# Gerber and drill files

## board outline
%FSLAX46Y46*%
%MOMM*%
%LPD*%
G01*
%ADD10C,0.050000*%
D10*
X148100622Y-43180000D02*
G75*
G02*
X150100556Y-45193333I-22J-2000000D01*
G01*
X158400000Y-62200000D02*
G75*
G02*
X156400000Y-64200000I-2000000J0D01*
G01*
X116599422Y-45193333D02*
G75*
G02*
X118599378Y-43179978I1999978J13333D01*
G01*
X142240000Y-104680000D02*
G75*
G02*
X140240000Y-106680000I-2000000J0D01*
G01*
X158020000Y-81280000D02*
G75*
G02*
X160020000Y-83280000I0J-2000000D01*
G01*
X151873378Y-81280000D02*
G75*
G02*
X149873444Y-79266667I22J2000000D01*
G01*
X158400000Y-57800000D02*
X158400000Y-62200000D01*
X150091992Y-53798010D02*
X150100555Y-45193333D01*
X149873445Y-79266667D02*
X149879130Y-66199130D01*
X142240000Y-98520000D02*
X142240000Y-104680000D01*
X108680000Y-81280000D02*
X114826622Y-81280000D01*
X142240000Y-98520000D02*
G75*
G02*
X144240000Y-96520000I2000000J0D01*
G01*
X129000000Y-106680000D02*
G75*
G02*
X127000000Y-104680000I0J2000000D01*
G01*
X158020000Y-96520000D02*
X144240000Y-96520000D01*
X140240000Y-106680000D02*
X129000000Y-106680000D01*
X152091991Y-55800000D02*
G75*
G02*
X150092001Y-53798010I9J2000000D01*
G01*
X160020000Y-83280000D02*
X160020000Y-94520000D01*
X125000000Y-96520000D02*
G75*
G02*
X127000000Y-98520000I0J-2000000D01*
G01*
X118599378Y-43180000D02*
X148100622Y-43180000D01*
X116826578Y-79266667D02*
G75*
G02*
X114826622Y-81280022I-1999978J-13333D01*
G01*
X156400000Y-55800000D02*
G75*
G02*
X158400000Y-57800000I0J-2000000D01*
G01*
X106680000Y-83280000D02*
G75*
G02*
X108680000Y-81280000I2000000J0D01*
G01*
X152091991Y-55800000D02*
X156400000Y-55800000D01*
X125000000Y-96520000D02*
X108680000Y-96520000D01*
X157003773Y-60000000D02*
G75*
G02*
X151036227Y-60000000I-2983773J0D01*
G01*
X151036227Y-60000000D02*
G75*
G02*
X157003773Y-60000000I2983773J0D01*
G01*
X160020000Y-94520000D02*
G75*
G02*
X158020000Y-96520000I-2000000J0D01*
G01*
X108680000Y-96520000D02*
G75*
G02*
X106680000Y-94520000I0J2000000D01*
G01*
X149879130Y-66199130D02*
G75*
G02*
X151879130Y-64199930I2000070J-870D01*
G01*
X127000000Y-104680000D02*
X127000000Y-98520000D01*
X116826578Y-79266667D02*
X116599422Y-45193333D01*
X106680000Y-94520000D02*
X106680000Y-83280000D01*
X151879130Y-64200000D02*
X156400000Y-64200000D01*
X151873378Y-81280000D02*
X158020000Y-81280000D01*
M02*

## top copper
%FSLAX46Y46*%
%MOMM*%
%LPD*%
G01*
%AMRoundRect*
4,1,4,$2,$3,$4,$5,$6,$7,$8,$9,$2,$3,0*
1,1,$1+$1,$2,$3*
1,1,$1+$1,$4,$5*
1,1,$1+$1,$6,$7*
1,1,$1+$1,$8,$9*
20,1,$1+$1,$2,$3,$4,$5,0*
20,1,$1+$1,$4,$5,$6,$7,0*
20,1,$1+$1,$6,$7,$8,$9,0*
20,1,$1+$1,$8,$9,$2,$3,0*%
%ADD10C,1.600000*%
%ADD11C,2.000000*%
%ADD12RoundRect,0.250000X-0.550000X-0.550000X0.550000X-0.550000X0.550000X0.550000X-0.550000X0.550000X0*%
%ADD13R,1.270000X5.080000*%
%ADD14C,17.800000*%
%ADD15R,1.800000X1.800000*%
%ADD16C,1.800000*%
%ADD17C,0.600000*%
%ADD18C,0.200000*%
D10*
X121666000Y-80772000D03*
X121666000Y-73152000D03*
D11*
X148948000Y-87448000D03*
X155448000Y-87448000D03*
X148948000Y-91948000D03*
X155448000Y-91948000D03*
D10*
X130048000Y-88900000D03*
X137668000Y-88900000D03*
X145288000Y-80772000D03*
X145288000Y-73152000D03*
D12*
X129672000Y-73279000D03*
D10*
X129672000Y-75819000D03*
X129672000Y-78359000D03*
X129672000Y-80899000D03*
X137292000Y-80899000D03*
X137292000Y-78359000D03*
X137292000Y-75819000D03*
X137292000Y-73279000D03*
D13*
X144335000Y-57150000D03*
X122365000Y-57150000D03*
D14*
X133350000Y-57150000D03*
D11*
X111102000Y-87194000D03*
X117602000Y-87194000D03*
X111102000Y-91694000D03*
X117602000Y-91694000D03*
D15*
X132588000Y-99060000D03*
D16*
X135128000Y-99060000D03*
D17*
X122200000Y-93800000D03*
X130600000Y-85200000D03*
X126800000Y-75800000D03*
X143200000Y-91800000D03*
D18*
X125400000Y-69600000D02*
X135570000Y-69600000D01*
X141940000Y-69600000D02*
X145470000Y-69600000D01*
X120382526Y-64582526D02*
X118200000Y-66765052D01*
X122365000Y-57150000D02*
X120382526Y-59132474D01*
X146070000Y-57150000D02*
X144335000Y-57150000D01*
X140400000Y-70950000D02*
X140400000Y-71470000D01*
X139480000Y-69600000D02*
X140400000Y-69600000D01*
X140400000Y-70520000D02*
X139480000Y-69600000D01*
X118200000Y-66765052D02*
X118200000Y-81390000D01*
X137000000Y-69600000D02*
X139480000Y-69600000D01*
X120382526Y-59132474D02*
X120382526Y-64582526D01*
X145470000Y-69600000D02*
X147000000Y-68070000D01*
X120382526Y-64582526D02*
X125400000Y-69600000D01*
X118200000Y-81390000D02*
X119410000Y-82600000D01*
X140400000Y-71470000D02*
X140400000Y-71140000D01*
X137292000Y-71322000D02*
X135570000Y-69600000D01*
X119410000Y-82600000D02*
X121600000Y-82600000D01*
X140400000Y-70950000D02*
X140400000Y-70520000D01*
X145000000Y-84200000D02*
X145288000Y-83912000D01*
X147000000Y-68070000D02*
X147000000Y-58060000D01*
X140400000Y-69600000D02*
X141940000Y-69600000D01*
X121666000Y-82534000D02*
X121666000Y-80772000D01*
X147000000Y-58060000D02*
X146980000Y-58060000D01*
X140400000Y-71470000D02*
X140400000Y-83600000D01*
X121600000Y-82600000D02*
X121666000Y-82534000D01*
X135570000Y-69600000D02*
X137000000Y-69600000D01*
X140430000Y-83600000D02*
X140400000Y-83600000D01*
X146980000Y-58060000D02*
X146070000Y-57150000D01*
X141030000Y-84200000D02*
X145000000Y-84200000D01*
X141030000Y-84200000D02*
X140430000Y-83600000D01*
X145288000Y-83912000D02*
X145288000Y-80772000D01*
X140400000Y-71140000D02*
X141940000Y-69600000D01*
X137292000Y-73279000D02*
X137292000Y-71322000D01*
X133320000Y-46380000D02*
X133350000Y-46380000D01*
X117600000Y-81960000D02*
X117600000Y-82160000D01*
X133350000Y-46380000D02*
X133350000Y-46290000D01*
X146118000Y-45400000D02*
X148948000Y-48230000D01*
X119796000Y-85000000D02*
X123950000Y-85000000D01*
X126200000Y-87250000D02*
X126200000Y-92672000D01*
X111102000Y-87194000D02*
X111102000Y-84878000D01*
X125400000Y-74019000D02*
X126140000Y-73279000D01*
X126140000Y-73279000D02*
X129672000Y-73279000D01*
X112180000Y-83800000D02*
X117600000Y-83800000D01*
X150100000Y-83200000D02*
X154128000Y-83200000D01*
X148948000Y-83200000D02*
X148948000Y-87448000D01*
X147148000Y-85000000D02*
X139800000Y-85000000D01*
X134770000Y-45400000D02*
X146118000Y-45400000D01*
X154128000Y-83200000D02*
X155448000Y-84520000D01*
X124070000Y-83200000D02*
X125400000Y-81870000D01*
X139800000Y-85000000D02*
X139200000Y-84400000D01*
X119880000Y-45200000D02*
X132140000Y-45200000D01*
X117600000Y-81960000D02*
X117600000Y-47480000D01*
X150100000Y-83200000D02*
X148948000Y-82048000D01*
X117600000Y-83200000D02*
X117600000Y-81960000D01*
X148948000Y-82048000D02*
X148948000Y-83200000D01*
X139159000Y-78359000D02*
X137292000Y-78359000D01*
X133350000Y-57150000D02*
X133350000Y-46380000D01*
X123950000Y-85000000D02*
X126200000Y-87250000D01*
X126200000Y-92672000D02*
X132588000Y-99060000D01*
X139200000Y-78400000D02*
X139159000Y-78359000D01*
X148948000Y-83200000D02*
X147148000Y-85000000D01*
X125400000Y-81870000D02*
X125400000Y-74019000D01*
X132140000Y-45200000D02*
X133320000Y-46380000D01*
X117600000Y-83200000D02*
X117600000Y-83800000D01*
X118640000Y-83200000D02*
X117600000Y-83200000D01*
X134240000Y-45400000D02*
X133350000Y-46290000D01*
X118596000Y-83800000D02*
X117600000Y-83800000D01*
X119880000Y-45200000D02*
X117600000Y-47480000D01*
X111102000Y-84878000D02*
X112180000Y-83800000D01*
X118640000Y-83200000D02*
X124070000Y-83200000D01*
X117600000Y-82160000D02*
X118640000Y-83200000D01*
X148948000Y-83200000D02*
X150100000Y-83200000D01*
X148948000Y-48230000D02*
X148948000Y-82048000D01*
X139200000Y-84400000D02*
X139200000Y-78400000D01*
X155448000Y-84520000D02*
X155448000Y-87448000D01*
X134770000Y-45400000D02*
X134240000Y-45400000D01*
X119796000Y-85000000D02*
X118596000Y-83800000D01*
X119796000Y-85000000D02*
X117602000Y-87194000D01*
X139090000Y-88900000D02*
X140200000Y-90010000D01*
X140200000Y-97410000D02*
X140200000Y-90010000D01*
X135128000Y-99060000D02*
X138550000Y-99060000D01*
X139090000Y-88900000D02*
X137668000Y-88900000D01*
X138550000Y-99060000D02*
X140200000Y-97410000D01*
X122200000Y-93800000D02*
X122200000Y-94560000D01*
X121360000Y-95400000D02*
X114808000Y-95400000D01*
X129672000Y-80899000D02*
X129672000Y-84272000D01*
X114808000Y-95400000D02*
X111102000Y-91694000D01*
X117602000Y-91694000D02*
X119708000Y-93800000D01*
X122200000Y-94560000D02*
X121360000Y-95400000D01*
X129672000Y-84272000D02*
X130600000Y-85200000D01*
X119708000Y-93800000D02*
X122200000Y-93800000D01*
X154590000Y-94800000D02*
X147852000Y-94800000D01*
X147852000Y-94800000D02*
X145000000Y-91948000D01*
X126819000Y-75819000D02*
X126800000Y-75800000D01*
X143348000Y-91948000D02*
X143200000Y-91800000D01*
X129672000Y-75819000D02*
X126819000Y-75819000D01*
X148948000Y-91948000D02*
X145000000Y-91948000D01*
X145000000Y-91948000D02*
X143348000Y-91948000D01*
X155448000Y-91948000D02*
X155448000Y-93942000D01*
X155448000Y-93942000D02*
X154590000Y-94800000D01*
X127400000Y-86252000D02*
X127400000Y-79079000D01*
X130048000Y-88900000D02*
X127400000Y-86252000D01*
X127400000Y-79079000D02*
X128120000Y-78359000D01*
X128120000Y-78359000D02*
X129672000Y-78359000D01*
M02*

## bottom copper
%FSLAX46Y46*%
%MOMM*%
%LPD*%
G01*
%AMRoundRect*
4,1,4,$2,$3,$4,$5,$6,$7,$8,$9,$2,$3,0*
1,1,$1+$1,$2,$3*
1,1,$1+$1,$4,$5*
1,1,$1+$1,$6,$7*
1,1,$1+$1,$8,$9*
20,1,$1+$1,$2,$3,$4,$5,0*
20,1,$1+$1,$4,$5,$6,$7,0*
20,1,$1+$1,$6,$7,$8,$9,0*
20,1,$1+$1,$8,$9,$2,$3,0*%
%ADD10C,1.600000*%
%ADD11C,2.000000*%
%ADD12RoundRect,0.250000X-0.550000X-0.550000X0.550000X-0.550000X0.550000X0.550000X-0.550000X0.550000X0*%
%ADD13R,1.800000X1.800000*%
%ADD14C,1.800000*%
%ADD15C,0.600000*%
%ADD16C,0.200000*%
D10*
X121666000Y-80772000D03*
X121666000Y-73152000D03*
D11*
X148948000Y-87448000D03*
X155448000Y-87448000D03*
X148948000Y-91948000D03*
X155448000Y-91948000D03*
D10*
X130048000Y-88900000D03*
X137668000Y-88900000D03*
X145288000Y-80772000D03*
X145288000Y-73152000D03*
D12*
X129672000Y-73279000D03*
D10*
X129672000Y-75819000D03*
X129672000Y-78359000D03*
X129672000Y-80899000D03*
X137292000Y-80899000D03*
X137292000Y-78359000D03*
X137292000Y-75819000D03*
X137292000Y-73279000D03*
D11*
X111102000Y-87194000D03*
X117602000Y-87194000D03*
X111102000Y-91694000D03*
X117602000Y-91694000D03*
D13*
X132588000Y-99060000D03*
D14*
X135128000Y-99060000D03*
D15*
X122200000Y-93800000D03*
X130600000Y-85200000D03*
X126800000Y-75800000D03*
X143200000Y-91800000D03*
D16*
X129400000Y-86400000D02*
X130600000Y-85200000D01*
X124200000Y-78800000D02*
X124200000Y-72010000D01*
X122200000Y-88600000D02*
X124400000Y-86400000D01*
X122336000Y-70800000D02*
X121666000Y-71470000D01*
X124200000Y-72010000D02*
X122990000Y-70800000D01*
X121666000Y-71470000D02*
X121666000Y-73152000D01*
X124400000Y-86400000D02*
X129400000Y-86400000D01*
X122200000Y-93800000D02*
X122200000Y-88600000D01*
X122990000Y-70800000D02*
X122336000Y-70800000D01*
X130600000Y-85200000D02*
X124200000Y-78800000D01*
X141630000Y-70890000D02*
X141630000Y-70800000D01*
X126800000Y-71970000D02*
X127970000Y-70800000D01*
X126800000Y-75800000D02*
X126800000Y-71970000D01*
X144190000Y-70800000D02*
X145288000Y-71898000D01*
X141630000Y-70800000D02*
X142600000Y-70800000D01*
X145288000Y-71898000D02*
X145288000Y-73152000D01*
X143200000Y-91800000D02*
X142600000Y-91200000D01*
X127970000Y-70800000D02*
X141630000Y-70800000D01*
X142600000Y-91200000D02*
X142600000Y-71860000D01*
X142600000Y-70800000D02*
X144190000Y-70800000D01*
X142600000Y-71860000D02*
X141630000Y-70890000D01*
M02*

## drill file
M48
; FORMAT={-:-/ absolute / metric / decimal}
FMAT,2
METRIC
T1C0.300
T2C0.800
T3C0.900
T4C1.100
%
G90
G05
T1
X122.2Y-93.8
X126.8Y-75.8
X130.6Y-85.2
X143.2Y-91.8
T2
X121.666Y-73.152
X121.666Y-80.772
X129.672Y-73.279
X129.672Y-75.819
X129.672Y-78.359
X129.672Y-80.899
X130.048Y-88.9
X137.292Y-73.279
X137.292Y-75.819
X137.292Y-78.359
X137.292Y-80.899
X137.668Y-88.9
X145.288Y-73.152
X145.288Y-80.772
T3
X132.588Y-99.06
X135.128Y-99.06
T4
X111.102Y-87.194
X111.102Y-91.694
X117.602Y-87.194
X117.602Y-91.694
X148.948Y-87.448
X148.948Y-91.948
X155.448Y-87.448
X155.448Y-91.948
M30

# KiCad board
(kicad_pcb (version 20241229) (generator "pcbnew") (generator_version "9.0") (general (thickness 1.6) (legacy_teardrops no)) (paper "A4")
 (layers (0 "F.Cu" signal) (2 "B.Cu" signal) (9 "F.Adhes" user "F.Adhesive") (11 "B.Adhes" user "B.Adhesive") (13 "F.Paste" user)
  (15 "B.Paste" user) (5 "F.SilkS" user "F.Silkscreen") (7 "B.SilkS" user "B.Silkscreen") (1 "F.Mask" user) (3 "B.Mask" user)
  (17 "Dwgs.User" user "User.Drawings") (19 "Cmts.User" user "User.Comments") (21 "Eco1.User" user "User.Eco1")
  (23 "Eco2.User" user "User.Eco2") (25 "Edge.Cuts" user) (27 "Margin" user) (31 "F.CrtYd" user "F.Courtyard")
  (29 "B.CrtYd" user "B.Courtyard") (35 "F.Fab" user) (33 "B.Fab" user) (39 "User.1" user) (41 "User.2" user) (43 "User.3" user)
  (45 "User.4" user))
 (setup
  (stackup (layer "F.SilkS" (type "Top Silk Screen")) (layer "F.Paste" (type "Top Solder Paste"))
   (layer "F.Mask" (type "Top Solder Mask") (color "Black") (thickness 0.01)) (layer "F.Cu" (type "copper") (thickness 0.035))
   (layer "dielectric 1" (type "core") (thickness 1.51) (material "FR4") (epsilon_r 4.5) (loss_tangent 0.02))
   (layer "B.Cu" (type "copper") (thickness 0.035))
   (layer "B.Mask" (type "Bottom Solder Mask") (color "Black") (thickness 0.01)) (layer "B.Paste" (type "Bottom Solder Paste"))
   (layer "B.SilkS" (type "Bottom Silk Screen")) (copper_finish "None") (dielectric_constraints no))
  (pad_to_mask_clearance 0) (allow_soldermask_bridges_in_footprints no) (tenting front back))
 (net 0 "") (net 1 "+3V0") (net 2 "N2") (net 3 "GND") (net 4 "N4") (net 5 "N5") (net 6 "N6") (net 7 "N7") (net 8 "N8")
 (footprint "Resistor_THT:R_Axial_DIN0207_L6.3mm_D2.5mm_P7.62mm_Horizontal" (layer "F.Cu") (at 121.666 80.772 90)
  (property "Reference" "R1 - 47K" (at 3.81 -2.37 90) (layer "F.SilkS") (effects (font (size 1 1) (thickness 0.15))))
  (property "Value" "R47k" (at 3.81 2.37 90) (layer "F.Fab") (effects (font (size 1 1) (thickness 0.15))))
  (pad "1" thru_hole circle (at 0 0 90) (size 1.6 1.6) (drill 0.8) (layers "*.Cu" "*.Mask") (remove_unused_layers no) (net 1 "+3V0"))
  (pad "2" thru_hole circle (at 7.62 0 90) (size 1.6 1.6) (drill 0.8) (layers "*.Cu" "*.Mask") (remove_unused_layers no) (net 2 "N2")))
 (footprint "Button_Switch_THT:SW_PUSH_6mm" (layer "F.Cu") (at 148.948 87.448)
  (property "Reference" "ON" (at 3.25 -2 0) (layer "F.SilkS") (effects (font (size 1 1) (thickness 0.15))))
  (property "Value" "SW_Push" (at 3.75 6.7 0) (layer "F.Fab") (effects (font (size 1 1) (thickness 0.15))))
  (pad "1" thru_hole circle (at 0 0 90) (size 2 2) (drill 1.1) (layers "*.Cu" "*.Mask") (remove_unused_layers no) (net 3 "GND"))
  (pad "1" thru_hole circle (at 6.5 0 90) (size 2 2) (drill 1.1) (layers "*.Cu" "*.Mask") (remove_unused_layers no) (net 3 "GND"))
  (pad "2" thru_hole circle (at 0 4.5 90) (size 2 2) (drill 1.1) (layers "*.Cu" "*.Mask") (remove_unused_layers no) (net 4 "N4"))
  (pad "2" thru_hole circle (at 6.5 4.5 90) (size 2 2) (drill 1.1) (layers "*.Cu" "*.Mask") (remove_unused_layers no) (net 4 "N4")))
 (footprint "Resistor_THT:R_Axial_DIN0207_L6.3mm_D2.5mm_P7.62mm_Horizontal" (layer "F.Cu") (at 130.048 88.9)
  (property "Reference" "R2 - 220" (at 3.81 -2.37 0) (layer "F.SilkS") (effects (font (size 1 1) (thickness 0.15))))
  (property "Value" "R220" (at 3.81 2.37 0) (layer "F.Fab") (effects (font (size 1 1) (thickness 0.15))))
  (pad "1" thru_hole circle (at 0 0) (size 1.6 1.6) (drill 0.8) (layers "*.Cu" "*.Mask") (remove_unused_layers no) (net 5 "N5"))
  (pad "2" thru_hole circle (at 7.62 0) (size 1.6 1.6) (drill 0.8) (layers "*.Cu" "*.Mask") (remove_unused_layers no) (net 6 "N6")))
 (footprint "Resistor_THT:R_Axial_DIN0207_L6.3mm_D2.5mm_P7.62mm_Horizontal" (layer "F.Cu") (at 145.288 80.772 90)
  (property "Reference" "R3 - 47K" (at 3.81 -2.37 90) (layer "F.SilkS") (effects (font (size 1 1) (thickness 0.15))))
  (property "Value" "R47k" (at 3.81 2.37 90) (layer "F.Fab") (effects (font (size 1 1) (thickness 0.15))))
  (pad "1" thru_hole circle (at 0 0 90) (size 1.6 1.6) (drill 0.8) (layers "*.Cu" "*.Mask") (remove_unused_layers no) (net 1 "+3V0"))
  (pad "2" thru_hole circle (at 7.62 0 90) (size 1.6 1.6) (drill 0.8) (layers "*.Cu" "*.Mask") (remove_unused_layers no) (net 4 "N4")))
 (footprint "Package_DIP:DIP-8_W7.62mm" (layer "F.Cu") (at 129.672 73.279)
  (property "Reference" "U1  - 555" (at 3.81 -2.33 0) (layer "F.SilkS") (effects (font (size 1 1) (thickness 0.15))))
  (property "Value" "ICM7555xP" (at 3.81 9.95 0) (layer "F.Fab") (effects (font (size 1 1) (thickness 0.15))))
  (pad "1" thru_hole roundrect (at 0 0) (size 1.6 1.6) (drill 0.8) (layers "*.Cu" "*.Mask") (remove_unused_layers no)
   (roundrect_rratio 0.15625) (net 3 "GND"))
  (pad "2" thru_hole circle (at 0 2.54) (size 1.6 1.6) (drill 0.8) (layers "*.Cu" "*.Mask") (remove_unused_layers no) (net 4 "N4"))
  (pad "3" thru_hole circle (at 0 5.08) (size 1.6 1.6) (drill 0.8) (layers "*.Cu" "*.Mask") (remove_unused_layers no) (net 5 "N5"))
  (pad "4" thru_hole circle (at 0 7.62) (size 1.6 1.6) (drill 0.8) (layers "*.Cu" "*.Mask") (remove_unused_layers no) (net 2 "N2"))
  (pad "5" thru_hole circle (at 7.62 7.62) (size 1.6 1.6) (drill 0.8) (layers "*.Cu" "*.Mask") (remove_unused_layers no) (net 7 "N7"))
  (pad "6" thru_hole circle (at 7.62 5.08) (size 1.6 1.6) (drill 0.8) (layers "*.Cu" "*.Mask") (remove_unused_layers no) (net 3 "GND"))
  (pad "7" thru_hole circle (at 7.62 2.54) (size 1.6 1.6) (drill 0.8) (layers "*.Cu" "*.Mask") (remove_unused_layers no) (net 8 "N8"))
  (pad "8" thru_hole circle (at 7.62 0) (size 1.6 1.6) (drill 0.8) (layers "*.Cu" "*.Mask") (remove_unused_layers no) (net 1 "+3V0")))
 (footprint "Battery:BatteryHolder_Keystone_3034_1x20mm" (layer "F.Cu") (at 133.35 57.15 180)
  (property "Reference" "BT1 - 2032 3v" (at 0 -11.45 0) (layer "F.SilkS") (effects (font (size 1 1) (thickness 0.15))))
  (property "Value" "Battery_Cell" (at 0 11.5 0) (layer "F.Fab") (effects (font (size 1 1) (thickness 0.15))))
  (pad "1" smd rect (at -10.985 0 180) (size 1.27 5.08) (layers "F.Cu" "F.Mask" "F.Paste") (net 1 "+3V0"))
  (pad "1" smd rect (at 10.985 0 180) (size 1.27 5.08) (layers "F.Cu" "F.Mask" "F.Paste") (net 1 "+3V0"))
  (pad "2" smd circle (at 0 0 180) (size 17.8 17.8) (layers "F.Cu" "F.Mask") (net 3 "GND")))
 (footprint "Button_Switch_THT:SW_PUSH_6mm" (layer "F.Cu") (at 111.102 87.194)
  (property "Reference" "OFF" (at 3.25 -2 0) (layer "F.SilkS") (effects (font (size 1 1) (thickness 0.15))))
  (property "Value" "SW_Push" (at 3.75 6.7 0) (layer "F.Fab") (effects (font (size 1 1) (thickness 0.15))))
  (pad "1" thru_hole circle (at 0 0 90) (size 2 2) (drill 1.1) (layers "*.Cu" "*.Mask") (remove_unused_layers no) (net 3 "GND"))
  (pad "1" thru_hole circle (at 6.5 0 90) (size 2 2) (drill 1.1) (layers "*.Cu" "*.Mask") (remove_unused_layers no) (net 3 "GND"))
  (pad "2" thru_hole circle (at 0 4.5 90) (size 2 2) (drill 1.1) (layers "*.Cu" "*.Mask") (remove_unused_layers no) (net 2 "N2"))
  (pad "2" thru_hole circle (at 6.5 4.5 90) (size 2 2) (drill 1.1) (layers "*.Cu" "*.Mask") (remove_unused_layers no) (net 2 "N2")))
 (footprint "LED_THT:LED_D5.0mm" (layer "F.Cu") (at 132.588 99.06)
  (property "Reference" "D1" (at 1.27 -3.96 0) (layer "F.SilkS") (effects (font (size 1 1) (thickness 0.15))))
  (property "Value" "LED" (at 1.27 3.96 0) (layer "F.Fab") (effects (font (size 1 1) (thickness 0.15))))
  (pad "1" thru_hole rect (at 0 0) (size 1.8 1.8) (drill 0.9) (layers "*.Cu" "*.Mask") (remove_unused_layers no) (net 3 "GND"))
  (pad "2" thru_hole circle (at 2.54 0) (size 1.8 1.8) (drill 0.9) (layers "*.Cu" "*.Mask") (remove_unused_layers no) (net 6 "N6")))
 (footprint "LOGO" (layer "B.Cu") (at 132.386961 57.005802 180)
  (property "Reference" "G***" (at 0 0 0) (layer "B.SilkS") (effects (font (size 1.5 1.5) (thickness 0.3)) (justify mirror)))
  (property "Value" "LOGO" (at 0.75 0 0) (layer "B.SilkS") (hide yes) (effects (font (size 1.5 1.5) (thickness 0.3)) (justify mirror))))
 (gr_arc (start 148.100622 43.18) (mid 149.519542 43.770508) (end 150.100578 45.193333) (stroke (width 0.05) (type default))
  (layer "Edge.Cuts"))
 (gr_arc (start 158.4 62.2) (mid 157.814214 63.614214) (end 156.4 64.2) (stroke (width 0.05) (type default)) (layer "Edge.Cuts"))
 (gr_arc (start 116.599422 45.193333) (mid 117.180457 43.7705) (end 118.599378 43.18) (stroke (width 0.05) (type default))
  (layer "Edge.Cuts"))
 (gr_arc (start 142.24 104.68) (mid 141.654214 106.094214) (end 140.24 106.68) (stroke (width 0.05) (type default)) (layer "Edge.Cuts"))
 (gr_arc (start 158.02 81.28) (mid 159.434214 81.865786) (end 160.02 83.28) (stroke (width 0.05) (type default)) (layer "Edge.Cuts"))
 (gr_arc (start 151.873378 81.28) (mid 150.454473 80.689484) (end 149.873422 79.266667) (stroke (width 0.05) (type default))
  (layer "Edge.Cuts"))
 (gr_line (start 158.4 57.8) (end 158.4 62.2) (stroke (width 0.05) (type default)) (layer "Edge.Cuts"))
 (gr_line (start 150.091992 53.79801) (end 150.100555 45.193333) (stroke (width 0.05) (type default)) (layer "Edge.Cuts"))
 (gr_line (start 149.873445 79.266667) (end 149.87913 66.19913) (stroke (width 0.05) (type default)) (layer "Edge.Cuts"))
 (gr_line (start 142.24 98.52) (end 142.24 104.68) (stroke (width 0.05) (type default)) (layer "Edge.Cuts"))
 (gr_line (start 108.68 81.28) (end 114.826622 81.28) (stroke (width 0.05) (type default)) (layer "Edge.Cuts"))
 (gr_arc (start 142.24 98.52) (mid 142.825786 97.105786) (end 144.24 96.52) (stroke (width 0.05) (type default)) (layer "Edge.Cuts"))
 (gr_arc (start 129 106.68) (mid 127.585786 106.094214) (end 127 104.68) (stroke (width 0.05) (type default)) (layer "Edge.Cuts"))
 (gr_line (start 158.02 96.52) (end 144.24 96.52) (stroke (width 0.05) (type default)) (layer "Edge.Cuts"))
 (gr_line (start 140.24 106.68) (end 129 106.68) (stroke (width 0.05) (type default)) (layer "Edge.Cuts"))
 (gr_arc (start 152.091991 55.8) (mid 150.67708 55.213507) (end 150.091992 53.79801) (stroke (width 0.05) (type default))
  (layer "Edge.Cuts"))
 (gr_line (start 160.02 83.28) (end 160.02 94.52) (stroke (width 0.05) (type default)) (layer "Edge.Cuts"))
 (gr_arc (start 125 96.52) (mid 126.414214 97.105786) (end 127 98.52) (stroke (width 0.05) (type default)) (layer "Edge.Cuts"))
 (gr_line (start 118.599378 43.18) (end 148.100622 43.18) (stroke (width 0.05) (type default)) (layer "Edge.Cuts"))
 (gr_arc (start 116.826578 79.266667) (mid 116.245542 80.689492) (end 114.826622 81.28) (stroke (width 0.05) (type default))
  (layer "Edge.Cuts"))
 (gr_arc (start 156.4 55.8) (mid 157.814214 56.385786) (end 158.4 57.8) (stroke (width 0.05) (type default)) (layer "Edge.Cuts"))
 (gr_arc (start 106.68 83.28) (mid 107.265786 81.865786) (end 108.68 81.28) (stroke (width 0.05) (type default)) (layer "Edge.Cuts"))
 (gr_line (start 152.091991 55.8) (end 156.4 55.8) (stroke (width 0.05) (type default)) (layer "Edge.Cuts"))
 (gr_line (start 125 96.52) (end 108.68 96.52) (stroke (width 0.05) (type default)) (layer "Edge.Cuts"))
 (gr_circle (center 154.02 60) (end 157 59.85) (stroke (width 0.05) (type default)) (fill no) (layer "Edge.Cuts"))
 (gr_arc (start 160.02 94.52) (mid 159.434214 95.934214) (end 158.02 96.52) (stroke (width 0.05) (type default)) (layer "Edge.Cuts"))
 (gr_arc (start 108.68 96.52) (mid 107.265786 95.934214) (end 106.68 94.52) (stroke (width 0.05) (type default)) (layer "Edge.Cuts"))
 (gr_arc (start 149.87913 66.19913) (mid 150.465226 64.785489) (end 151.87913 64.2) (stroke (width 0.05) (type default)) (layer "Edge.Cuts"))
 (gr_line (start 127 104.68) (end 127 98.52) (stroke (width 0.05) (type default)) (layer "Edge.Cuts"))
 (gr_line (start 116.826578 79.266667) (end 116.599422 45.193333) (stroke (width 0.05) (type default)) (layer "Edge.Cuts"))
 (gr_line (start 106.68 94.52) (end 106.68 83.28) (stroke (width 0.05) (type default)) (layer "Edge.Cuts"))
 (gr_line (start 151.87913 64.2) (end 156.4 64.2) (stroke (width 0.05) (type default)) (layer "Edge.Cuts"))
 (gr_line (start 151.873378 81.28) (end 158.02 81.28) (stroke (width 0.05) (type default)) (layer "Edge.Cuts"))
 (segment (start 125.4 69.6) (end 135.57 69.6) (width 0.2) (layer "F.Cu") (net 1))
 (segment (start 141.94 69.6) (end 145.47 69.6) (width 0.2) (layer "F.Cu") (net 1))
 (segment (start 120.382526 64.582526) (end 118.2 66.765052) (width 0.2) (layer "F.Cu") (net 1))
 (segment (start 122.365 57.15) (end 120.382526 59.132474) (width 0.2) (layer "F.Cu") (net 1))
 (segment (start 146.07 57.15) (end 144.335 57.15) (width 0.2) (layer "F.Cu") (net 1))
 (segment (start 140.4 70.95) (end 140.4 71.47) (width 0.2) (layer "F.Cu") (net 1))
 (segment (start 139.48 69.6) (end 140.4 69.6) (width 0.2) (layer "F.Cu") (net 1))
 (segment (start 140.4 70.52) (end 139.48 69.6) (width 0.2) (layer "F.Cu") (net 1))
 (segment (start 118.2 66.765052) (end 118.2 81.39) (width 0.2) (layer "F.Cu") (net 1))
 (segment (start 137 69.6) (end 139.48 69.6) (width 0.2) (layer "F.Cu") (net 1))
 (segment (start 120.382526 59.132474) (end 120.382526 64.582526) (width 0.2) (layer "F.Cu") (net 1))
 (segment (start 145.47 69.6) (end 147 68.07) (width 0.2) (layer "F.Cu") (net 1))
 (segment (start 120.382526 64.582526) (end 125.4 69.6) (width 0.2) (layer "F.Cu") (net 1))
 (segment (start 118.2 81.39) (end 119.41 82.6) (width 0.2) (layer "F.Cu") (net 1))
 (segment (start 140.4 71.47) (end 140.4 71.14) (width 0.2) (layer "F.Cu") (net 1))
 (segment (start 137.292 71.322) (end 135.57 69.6) (width 0.2) (layer "F.Cu") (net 1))
 (segment (start 119.41 82.6) (end 121.6 82.6) (width 0.2) (layer "F.Cu") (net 1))
 (segment (start 140.4 70.95) (end 140.4 70.52) (width 0.2) (layer "F.Cu") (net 1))
 (segment (start 145 84.2) (end 145.288 83.912) (width 0.2) (layer "F.Cu") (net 1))
 (segment (start 147 68.07) (end 147 58.06) (width 0.2) (layer "F.Cu") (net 1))
 (segment (start 140.4 69.6) (end 141.94 69.6) (width 0.2) (layer "F.Cu") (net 1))
 (segment (start 121.666 82.534) (end 121.666 80.772) (width 0.2) (layer "F.Cu") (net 1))
 (segment (start 147 58.06) (end 146.98 58.06) (width 0.2) (layer "F.Cu") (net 1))
 (segment (start 140.4 71.47) (end 140.4 83.6) (width 0.2) (layer "F.Cu") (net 1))
 (segment (start 121.6 82.6) (end 121.666 82.534) (width 0.2) (layer "F.Cu") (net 1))
 (segment (start 135.57 69.6) (end 137 69.6) (width 0.2) (layer "F.Cu") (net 1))
 (segment (start 140.43 83.6) (end 140.4 83.6) (width 0.2) (layer "F.Cu") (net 1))
 (segment (start 146.98 58.06) (end 146.07 57.15) (width 0.2) (layer "F.Cu") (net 1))
 (segment (start 141.03 84.2) (end 145 84.2) (width 0.2) (layer "F.Cu") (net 1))
 (segment (start 141.03 84.2) (end 140.43 83.6) (width 0.2) (layer "F.Cu") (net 1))
 (segment (start 145.288 83.912) (end 145.288 80.772) (width 0.2) (layer "F.Cu") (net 1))
 (segment (start 140.4 71.14) (end 141.94 69.6) (width 0.2) (layer "F.Cu") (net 1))
 (segment (start 137.292 73.279) (end 137.292 71.322) (width 0.2) (layer "F.Cu") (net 1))
 (segment (start 133.32 46.38) (end 133.35 46.38) (width 0.2) (layer "F.Cu") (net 3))
 (segment (start 117.6 81.96) (end 117.6 82.16) (width 0.2) (layer "F.Cu") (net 3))
 (segment (start 133.35 46.38) (end 133.35 46.29) (width 0.2) (layer "F.Cu") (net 3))
 (segment (start 146.118 45.4) (end 148.948 48.23) (width 0.2) (layer "F.Cu") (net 3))
 (segment (start 119.796 85) (end 123.95 85) (width 0.2) (layer "F.Cu") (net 3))
 (segment (start 126.2 87.25) (end 126.2 92.672) (width 0.2) (layer "F.Cu") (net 3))
 (segment (start 111.102 87.194) (end 111.102 84.878) (width 0.2) (layer "F.Cu") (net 3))
 (segment (start 125.4 74.019) (end 126.14 73.279) (width 0.2) (layer "F.Cu") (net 3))
 (segment (start 126.14 73.279) (end 129.672 73.279) (width 0.2) (layer "F.Cu") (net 3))
 (segment (start 112.18 83.8) (end 117.6 83.8) (width 0.2) (layer "F.Cu") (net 3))
 (segment (start 150.1 83.2) (end 154.128 83.2) (width 0.2) (layer "F.Cu") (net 3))
 (segment (start 148.948 83.2) (end 148.948 87.448) (width 0.2) (layer "F.Cu") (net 3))
 (segment (start 147.148 85) (end 139.8 85) (width 0.2) (layer "F.Cu") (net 3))
 (segment (start 134.77 45.4) (end 146.118 45.4) (width 0.2) (layer "F.Cu") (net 3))
 (segment (start 154.128 83.2) (end 155.448 84.52) (width 0.2) (layer "F.Cu") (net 3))
 (segment (start 124.07 83.2) (end 125.4 81.87) (width 0.2) (layer "F.Cu") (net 3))
 (segment (start 139.8 85) (end 139.2 84.4) (width 0.2) (layer "F.Cu") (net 3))
 (segment (start 119.88 45.2) (end 132.14 45.2) (width 0.2) (layer "F.Cu") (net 3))
 (segment (start 117.6 81.96) (end 117.6 47.48) (width 0.2) (layer "F.Cu") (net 3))
 (segment (start 150.1 83.2) (end 148.948 82.048) (width 0.2) (layer "F.Cu") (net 3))
 (segment (start 117.6 83.2) (end 117.6 81.96) (width 0.2) (layer "F.Cu") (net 3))
 (segment (start 148.948 82.048) (end 148.948 83.2) (width 0.2) (layer "F.Cu") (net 3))
 (segment (start 139.159 78.359) (end 137.292 78.359) (width 0.2) (layer "F.Cu") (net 3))
 (segment (start 133.35 57.15) (end 133.35 46.38) (width 0.2) (layer "F.Cu") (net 3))
 (segment (start 123.95 85) (end 126.2 87.25) (width 0.2) (layer "F.Cu") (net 3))
 (segment (start 126.2 92.672) (end 132.588 99.06) (width 0.2) (layer "F.Cu") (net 3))
 (segment (start 139.2 78.4) (end 139.159 78.359) (width 0.2) (layer "F.Cu") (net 3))
 (segment (start 148.948 83.2) (end 147.148 85) (width 0.2) (layer "F.Cu") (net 3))
 (segment (start 125.4 81.87) (end 125.4 74.019) (width 0.2) (layer "F.Cu") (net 3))
 (segment (start 132.14 45.2) (end 133.32 46.38) (width 0.2) (layer "F.Cu") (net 3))
 (segment (start 117.6 83.2) (end 117.6 83.8) (width 0.2) (layer "F.Cu") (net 3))
 (segment (start 118.64 83.2) (end 117.6 83.2) (width 0.2) (layer "F.Cu") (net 3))
 (segment (start 134.24 45.4) (end 133.35 46.29) (width 0.2) (layer "F.Cu") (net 3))
 (segment (start 118.596 83.8) (end 117.6 83.8) (width 0.2) (layer "F.Cu") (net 3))
 (segment (start 119.88 45.2) (end 117.6 47.48) (width 0.2) (layer "F.Cu") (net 3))
 (segment (start 111.102 84.878) (end 112.18 83.8) (width 0.2) (layer "F.Cu") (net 3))
 (segment (start 118.64 83.2) (end 124.07 83.2) (width 0.2) (layer "F.Cu") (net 3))
 (segment (start 117.6 82.16) (end 118.64 83.2) (width 0.2) (layer "F.Cu") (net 3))
 (segment (start 148.948 83.2) (end 150.1 83.2) (width 0.2) (layer "F.Cu") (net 3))
 (segment (start 148.948 48.23) (end 148.948 82.048) (width 0.2) (layer "F.Cu") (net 3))
 (segment (start 139.2 84.4) (end 139.2 78.4) (width 0.2) (layer "F.Cu") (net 3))
 (segment (start 155.448 84.52) (end 155.448 87.448) (width 0.2) (layer "F.Cu") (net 3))
 (segment (start 134.77 45.4) (end 134.24 45.4) (width 0.2) (layer "F.Cu") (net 3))
 (segment (start 119.796 85) (end 118.596 83.8) (width 0.2) (layer "F.Cu") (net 3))
 (segment (start 119.796 85) (end 117.602 87.194) (width 0.2) (layer "F.Cu") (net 3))
 (segment (start 139.09 88.9) (end 140.2 90.01) (width 0.2) (layer "F.Cu") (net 6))
 (segment (start 140.2 97.41) (end 140.2 90.01) (width 0.2) (layer "F.Cu") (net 6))
 (segment (start 135.128 99.06) (end 138.55 99.06) (width 0.2) (layer "F.Cu") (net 6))
 (segment (start 139.09 88.9) (end 137.668 88.9) (width 0.2) (layer "F.Cu") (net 6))
 (segment (start 138.55 99.06) (end 140.2 97.41) (width 0.2) (layer "F.Cu") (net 6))
 (segment (start 122.2 93.8) (end 122.2 94.56) (width 0.2) (layer "F.Cu") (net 2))
 (segment (start 121.36 95.4) (end 114.808 95.4) (width 0.2) (layer "F.Cu") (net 2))
 (segment (start 129.672 80.899) (end 129.672 84.272) (width 0.2) (layer "F.Cu") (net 2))
 (segment (start 114.808 95.4) (end 111.102 91.694) (width 0.2) (layer "F.Cu") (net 2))
 (segment (start 117.602 91.694) (end 119.708 93.8) (width 0.2) (layer "F.Cu") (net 2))
 (segment (start 122.2 94.56) (end 121.36 95.4) (width 0.2) (layer "F.Cu") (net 2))
 (segment (start 129.672 84.272) (end 130.6 85.2) (width 0.2) (layer "F.Cu") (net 2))
 (segment (start 119.708 93.8) (end 122.2 93.8) (width 0.2) (layer "F.Cu") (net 2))
 (via (at 122.2 93.8) (size 0.6) (drill 0.3) (layers "F.Cu" "B.Cu") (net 2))
 (via (at 130.6 85.2) (size 0.6) (drill 0.3) (layers "F.Cu" "B.Cu") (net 2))
 (segment (start 129.4 86.4) (end 130.6 85.2) (width 0.2) (layer "B.Cu") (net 2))
 (segment (start 124.2 78.8) (end 124.2 72.01) (width 0.2) (layer "B.Cu") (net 2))
 (segment (start 122.2 88.6) (end 124.4 86.4) (width 0.2) (layer "B.Cu") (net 2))
 (segment (start 122.336 70.8) (end 121.666 71.47) (width 0.2) (layer "B.Cu") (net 2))
 (segment (start 124.2 72.01) (end 122.99 70.8) (width 0.2) (layer "B.Cu") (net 2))
 (segment (start 121.666 71.47) (end 121.666 73.152) (width 0.2) (layer "B.Cu") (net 2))
 (segment (start 124.4 86.4) (end 129.4 86.4) (width 0.2) (layer "B.Cu") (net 2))
 (segment (start 122.2 93.8) (end 122.2 88.6) (width 0.2) (layer "B.Cu") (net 2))
 (segment (start 122.99 70.8) (end 122.336 70.8) (width 0.2) (layer "B.Cu") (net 2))
 (segment (start 130.6 85.2) (end 124.2 78.8) (width 0.2) (layer "B.Cu") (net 2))
 (segment (start 154.59 94.8) (end 147.852 94.8) (width 0.2) (layer "F.Cu") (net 4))
 (segment (start 147.852 94.8) (end 145 91.948) (width 0.2) (layer "F.Cu") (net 4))
 (segment (start 126.819 75.819) (end 126.8 75.8) (width 0.2) (layer "F.Cu") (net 4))
 (segment (start 143.348 91.948) (end 143.2 91.8) (width 0.2) (layer "F.Cu") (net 4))
 (segment (start 129.672 75.819) (end 126.819 75.819) (width 0.2) (layer "F.Cu") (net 4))
 (segment (start 148.948 91.948) (end 145 91.948) (width 0.2) (layer "F.Cu") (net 4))
 (segment (start 145 91.948) (end 143.348 91.948) (width 0.2) (layer "F.Cu") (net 4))
 (segment (start 155.448 91.948) (end 155.448 93.942) (width 0.2) (layer "F.Cu") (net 4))
 (segment (start 155.448 93.942) (end 154.59 94.8) (width 0.2) (layer "F.Cu") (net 4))
 (via (at 126.8 75.8) (size 0.6) (drill 0.3) (layers "F.Cu" "B.Cu") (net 4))
 (via (at 143.2 91.8) (size 0.6) (drill 0.3) (layers "F.Cu" "B.Cu") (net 4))
 (segment (start 141.63 70.89) (end 141.63 70.8) (width 0.2) (layer "B.Cu") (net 4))
 (segment (start 126.8 71.97) (end 127.97 70.8) (width 0.2) (layer "B.Cu") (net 4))
 (segment (start 126.8 75.8) (end 126.8 71.97) (width 0.2) (layer "B.Cu") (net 4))
 (segment (start 144.19 70.8) (end 145.288 71.898) (width 0.2) (layer "B.Cu") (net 4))
 (segment (start 141.63 70.8) (end 142.6 70.8) (width 0.2) (layer "B.Cu") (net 4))
 (segment (start 145.288 71.898) (end 145.288 73.152) (width 0.2) (layer "B.Cu") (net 4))
 (segment (start 143.2 91.8) (end 142.6 91.2) (width 0.2) (layer "B.Cu") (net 4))
 (segment (start 127.97 70.8) (end 141.63 70.8) (width 0.2) (layer "B.Cu") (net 4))
 (segment (start 142.6 91.2) (end 142.6 71.86) (width 0.2) (layer "B.Cu") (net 4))
 (segment (start 142.6 70.8) (end 144.19 70.8) (width 0.2) (layer "B.Cu") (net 4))
 (segment (start 142.6 71.86) (end 141.63 70.89) (width 0.2) (layer "B.Cu") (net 4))
 (segment (start 127.4 86.252) (end 127.4 79.079) (width 0.2) (layer "F.Cu") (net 5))
 (segment (start 130.048 88.9) (end 127.4 86.252) (width 0.2) (layer "F.Cu") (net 5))
 (segment (start 127.4 79.079) (end 128.12 78.359) (width 0.2) (layer "F.Cu") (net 5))
 (segment (start 128.12 78.359) (end 129.672 78.359) (width 0.2) (layer "F.Cu") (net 5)))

